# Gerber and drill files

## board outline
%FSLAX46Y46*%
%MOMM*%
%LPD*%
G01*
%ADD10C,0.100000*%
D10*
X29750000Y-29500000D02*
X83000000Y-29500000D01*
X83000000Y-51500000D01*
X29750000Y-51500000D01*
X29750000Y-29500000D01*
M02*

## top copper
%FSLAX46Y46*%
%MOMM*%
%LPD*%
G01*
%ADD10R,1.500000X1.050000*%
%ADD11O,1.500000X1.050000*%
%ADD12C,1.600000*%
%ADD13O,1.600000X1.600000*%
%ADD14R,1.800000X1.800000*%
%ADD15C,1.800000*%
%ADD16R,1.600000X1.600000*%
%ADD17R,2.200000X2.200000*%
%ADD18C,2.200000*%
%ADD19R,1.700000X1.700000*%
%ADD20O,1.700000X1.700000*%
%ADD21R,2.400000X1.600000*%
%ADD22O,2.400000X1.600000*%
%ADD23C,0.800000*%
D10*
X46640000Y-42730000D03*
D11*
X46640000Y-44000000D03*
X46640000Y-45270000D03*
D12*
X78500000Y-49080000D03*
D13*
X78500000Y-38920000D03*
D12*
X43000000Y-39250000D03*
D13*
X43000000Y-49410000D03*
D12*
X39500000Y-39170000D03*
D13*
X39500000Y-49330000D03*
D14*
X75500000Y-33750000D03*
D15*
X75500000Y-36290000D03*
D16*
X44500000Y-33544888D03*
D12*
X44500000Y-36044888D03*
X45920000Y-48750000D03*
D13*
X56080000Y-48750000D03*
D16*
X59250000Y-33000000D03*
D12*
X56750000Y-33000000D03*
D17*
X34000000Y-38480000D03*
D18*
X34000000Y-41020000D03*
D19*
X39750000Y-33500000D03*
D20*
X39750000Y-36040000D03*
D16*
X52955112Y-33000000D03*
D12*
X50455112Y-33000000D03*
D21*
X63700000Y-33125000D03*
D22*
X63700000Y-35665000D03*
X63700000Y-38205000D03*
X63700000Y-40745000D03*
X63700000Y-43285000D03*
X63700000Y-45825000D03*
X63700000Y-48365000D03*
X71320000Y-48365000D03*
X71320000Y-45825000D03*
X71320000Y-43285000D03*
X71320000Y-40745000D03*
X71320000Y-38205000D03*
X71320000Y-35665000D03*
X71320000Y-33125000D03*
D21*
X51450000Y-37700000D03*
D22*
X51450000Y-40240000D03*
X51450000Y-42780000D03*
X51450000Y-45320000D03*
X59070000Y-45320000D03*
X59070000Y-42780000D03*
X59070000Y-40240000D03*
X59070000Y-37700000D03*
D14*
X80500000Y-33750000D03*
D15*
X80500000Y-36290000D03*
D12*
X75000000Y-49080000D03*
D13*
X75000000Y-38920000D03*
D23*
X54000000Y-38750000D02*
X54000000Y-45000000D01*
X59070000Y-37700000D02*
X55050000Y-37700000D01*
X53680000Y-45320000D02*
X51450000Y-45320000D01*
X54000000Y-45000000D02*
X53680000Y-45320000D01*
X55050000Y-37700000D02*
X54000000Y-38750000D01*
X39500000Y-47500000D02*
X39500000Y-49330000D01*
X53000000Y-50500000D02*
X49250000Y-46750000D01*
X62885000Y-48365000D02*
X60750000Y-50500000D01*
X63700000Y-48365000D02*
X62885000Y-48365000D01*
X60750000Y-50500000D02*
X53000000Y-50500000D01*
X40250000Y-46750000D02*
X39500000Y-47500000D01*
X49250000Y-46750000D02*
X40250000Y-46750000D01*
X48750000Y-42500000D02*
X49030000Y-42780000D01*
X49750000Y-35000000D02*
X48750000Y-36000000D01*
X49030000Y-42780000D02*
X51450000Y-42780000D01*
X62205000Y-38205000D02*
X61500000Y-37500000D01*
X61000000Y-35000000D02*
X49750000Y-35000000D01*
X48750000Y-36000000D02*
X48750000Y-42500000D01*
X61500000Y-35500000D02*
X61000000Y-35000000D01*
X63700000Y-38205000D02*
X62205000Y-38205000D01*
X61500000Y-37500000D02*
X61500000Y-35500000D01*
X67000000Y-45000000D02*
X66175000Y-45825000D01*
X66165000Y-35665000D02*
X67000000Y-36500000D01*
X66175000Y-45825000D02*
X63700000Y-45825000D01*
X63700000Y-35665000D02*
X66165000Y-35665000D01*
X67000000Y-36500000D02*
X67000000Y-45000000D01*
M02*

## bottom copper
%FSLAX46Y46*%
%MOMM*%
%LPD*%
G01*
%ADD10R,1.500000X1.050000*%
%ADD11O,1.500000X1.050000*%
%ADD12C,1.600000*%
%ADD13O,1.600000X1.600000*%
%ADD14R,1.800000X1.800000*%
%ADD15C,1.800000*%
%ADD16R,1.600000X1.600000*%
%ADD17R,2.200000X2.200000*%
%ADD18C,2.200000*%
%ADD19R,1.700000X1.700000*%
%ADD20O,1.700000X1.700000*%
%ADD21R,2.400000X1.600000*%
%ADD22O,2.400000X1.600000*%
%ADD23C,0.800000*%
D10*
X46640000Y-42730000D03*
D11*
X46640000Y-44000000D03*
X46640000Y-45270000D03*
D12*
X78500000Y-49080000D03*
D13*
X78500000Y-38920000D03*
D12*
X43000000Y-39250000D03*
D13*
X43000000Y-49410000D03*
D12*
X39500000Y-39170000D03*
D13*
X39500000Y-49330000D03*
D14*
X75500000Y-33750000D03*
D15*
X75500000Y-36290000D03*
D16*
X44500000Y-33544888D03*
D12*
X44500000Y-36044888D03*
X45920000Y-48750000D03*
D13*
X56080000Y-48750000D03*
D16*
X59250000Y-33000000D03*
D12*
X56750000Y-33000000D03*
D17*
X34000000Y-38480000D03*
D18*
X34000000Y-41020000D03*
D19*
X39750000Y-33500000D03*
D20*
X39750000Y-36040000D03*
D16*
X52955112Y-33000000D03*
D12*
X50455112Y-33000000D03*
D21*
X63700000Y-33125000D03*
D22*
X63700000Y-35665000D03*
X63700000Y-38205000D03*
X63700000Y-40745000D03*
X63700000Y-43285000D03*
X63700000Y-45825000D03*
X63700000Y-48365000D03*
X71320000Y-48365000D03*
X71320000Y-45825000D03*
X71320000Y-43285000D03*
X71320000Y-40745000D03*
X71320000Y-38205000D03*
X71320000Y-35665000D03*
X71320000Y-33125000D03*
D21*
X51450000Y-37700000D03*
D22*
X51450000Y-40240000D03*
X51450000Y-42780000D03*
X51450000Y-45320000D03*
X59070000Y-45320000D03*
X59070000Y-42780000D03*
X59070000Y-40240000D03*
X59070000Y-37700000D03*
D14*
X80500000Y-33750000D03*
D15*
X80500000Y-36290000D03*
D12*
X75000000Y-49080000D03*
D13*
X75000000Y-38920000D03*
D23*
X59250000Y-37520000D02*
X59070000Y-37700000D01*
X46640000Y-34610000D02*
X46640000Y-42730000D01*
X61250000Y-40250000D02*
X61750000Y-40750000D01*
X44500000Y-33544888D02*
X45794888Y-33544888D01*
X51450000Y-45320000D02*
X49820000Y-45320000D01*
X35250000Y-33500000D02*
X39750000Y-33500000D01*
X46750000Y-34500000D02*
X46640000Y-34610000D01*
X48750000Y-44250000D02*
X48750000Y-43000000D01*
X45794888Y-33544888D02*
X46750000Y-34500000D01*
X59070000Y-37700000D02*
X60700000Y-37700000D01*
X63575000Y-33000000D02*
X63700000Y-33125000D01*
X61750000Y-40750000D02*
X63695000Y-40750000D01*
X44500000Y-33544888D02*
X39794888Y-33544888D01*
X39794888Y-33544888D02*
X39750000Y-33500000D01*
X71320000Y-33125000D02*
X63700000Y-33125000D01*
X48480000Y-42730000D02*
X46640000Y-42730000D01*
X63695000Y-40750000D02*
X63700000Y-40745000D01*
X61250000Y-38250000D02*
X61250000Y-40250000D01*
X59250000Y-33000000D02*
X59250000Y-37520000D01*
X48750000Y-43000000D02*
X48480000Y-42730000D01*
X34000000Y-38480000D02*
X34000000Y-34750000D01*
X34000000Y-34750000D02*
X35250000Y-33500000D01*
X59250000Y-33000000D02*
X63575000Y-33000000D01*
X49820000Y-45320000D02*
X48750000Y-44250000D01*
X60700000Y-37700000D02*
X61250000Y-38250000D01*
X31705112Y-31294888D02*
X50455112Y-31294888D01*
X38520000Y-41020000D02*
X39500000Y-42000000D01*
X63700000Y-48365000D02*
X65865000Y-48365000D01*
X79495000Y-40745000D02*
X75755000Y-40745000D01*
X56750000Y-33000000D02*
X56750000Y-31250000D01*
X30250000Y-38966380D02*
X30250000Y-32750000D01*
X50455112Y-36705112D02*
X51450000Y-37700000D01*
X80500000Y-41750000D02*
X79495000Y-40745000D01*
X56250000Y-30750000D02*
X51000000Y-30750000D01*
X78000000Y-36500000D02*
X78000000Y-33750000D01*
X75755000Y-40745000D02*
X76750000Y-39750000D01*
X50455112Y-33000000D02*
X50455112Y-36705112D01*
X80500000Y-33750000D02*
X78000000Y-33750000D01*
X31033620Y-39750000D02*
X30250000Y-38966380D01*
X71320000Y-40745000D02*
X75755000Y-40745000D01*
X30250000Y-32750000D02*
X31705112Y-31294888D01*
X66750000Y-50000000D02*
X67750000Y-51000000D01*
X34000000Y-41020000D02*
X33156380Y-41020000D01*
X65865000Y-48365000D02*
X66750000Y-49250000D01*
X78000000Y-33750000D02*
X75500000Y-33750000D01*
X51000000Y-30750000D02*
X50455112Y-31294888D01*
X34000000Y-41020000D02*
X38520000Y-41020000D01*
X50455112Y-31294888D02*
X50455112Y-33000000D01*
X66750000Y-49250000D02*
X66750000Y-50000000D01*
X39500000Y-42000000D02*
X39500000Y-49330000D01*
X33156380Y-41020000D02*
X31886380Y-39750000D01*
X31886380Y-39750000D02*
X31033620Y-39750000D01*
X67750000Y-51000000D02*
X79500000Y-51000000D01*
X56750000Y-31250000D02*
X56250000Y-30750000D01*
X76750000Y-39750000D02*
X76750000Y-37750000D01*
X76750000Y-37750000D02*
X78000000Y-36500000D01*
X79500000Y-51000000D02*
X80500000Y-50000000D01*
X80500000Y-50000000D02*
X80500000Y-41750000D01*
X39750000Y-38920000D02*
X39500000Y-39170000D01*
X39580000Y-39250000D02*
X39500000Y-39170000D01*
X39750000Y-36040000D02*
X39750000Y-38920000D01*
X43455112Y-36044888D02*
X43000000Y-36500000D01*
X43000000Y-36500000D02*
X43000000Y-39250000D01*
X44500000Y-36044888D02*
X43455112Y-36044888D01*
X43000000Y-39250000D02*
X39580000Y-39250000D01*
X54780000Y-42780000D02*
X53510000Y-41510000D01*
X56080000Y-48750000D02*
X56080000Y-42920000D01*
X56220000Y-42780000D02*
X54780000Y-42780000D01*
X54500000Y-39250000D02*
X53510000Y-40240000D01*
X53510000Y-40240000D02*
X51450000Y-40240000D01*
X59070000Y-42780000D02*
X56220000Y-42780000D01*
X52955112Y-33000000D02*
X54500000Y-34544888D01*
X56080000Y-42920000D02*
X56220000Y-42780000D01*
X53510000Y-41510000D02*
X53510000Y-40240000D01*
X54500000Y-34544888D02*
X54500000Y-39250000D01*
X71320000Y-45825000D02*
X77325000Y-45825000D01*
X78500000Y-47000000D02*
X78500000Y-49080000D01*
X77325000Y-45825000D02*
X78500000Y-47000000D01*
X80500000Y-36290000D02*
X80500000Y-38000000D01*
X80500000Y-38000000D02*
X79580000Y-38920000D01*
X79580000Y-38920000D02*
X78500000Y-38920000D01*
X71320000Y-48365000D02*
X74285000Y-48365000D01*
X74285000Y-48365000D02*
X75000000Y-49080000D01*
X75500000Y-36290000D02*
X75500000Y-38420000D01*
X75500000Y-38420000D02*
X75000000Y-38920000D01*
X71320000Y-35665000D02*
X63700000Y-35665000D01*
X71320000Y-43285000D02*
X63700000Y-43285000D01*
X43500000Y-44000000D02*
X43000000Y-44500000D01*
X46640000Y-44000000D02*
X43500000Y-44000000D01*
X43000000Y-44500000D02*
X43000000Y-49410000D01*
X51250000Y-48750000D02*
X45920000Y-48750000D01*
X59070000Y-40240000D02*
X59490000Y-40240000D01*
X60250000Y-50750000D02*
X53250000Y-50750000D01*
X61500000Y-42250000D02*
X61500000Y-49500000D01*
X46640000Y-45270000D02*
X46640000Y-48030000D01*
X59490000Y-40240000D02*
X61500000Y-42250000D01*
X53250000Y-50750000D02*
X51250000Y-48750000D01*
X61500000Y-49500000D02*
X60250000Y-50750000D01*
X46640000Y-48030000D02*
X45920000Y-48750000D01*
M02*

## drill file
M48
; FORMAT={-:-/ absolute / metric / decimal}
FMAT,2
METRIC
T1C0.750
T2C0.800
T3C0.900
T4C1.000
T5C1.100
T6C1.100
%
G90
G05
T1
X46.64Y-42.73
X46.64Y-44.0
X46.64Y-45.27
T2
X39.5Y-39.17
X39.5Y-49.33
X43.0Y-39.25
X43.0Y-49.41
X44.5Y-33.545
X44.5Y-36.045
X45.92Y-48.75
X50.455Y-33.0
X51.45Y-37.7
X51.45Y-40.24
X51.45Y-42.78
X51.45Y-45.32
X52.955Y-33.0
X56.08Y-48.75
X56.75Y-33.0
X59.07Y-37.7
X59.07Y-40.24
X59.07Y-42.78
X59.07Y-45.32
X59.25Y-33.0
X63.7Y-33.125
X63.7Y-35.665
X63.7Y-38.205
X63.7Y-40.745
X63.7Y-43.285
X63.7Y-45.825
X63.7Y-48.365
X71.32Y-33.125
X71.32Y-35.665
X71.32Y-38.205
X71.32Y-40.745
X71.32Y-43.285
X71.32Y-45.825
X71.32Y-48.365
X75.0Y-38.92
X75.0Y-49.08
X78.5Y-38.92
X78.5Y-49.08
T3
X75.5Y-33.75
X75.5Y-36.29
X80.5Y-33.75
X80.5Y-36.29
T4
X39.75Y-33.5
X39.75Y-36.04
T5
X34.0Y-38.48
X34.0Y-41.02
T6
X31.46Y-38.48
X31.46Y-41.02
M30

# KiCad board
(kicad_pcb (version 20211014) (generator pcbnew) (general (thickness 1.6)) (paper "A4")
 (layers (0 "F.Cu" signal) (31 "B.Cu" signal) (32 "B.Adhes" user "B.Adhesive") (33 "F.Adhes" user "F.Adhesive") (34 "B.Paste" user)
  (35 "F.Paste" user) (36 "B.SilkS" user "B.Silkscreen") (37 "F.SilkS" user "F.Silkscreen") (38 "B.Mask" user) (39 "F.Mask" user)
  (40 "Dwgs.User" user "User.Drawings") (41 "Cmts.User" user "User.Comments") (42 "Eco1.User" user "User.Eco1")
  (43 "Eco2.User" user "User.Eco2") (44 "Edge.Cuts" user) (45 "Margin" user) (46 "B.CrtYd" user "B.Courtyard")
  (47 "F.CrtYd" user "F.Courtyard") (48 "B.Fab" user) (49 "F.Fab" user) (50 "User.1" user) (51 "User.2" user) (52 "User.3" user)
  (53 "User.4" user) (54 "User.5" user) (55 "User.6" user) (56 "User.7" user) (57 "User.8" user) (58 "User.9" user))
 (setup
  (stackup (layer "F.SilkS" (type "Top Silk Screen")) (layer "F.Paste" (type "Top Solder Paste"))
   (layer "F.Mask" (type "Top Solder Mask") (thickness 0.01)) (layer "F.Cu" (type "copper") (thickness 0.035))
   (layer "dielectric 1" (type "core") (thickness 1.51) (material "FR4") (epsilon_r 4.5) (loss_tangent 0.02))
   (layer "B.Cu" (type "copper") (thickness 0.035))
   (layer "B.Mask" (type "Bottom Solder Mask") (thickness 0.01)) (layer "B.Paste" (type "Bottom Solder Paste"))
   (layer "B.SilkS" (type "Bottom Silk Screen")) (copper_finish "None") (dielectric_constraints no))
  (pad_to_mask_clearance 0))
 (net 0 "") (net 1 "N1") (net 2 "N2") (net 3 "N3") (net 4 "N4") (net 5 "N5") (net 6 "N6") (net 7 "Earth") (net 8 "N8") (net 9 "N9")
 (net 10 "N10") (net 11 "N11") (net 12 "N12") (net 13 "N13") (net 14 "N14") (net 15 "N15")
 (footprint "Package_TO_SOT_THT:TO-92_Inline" (layer "F.Cu") (at 46.64 42.73 -90)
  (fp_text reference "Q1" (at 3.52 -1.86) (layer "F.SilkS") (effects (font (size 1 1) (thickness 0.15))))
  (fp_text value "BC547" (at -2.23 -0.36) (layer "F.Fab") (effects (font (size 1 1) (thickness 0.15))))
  (pad "1" thru_hole rect locked (at 0 0 270) (size 1.05 1.5) (drill 0.75) (layers *.Cu *.Mask) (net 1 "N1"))
  (pad "2" thru_hole oval locked (at 1.27 0 270) (size 1.05 1.5) (drill 0.75) (layers *.Cu *.Mask) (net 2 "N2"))
  (pad "3" thru_hole oval locked (at 2.54 0 270) (size 1.05 1.5) (drill 0.75) (layers *.Cu *.Mask) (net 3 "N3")))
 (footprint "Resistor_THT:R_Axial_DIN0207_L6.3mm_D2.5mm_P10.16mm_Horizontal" (layer "F.Cu") (at 78.5 49.08 90)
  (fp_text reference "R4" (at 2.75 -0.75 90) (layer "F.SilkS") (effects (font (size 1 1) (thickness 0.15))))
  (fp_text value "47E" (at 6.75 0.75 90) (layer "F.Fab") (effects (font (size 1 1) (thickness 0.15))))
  (pad "1" thru_hole circle locked (at 0 0 90) (size 1.6 1.6) (drill 0.8) (layers *.Cu *.Mask) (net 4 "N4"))
  (pad "2" thru_hole oval locked (at 10.16 0 90) (size 1.6 1.6) (drill 0.8) (layers *.Cu *.Mask) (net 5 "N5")))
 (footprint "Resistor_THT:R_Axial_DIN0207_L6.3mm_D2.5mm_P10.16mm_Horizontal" (layer "F.Cu") (at 43 39.25 -90)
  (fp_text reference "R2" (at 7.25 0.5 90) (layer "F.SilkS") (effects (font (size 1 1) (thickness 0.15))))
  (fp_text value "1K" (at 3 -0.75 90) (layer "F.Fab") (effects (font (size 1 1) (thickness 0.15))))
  (pad "1" thru_hole circle locked (at 0 0 270) (size 1.6 1.6) (drill 0.8) (layers *.Cu *.Mask) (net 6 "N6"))
  (pad "2" thru_hole oval locked (at 10.16 0 270) (size 1.6 1.6) (drill 0.8) (layers *.Cu *.Mask) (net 2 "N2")))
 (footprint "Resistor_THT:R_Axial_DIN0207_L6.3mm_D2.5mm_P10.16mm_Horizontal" (layer "F.Cu") (at 39.5 39.17 -90)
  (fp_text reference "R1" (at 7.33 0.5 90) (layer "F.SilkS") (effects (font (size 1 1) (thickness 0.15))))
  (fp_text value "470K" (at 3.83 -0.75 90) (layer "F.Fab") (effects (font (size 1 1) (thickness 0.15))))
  (pad "1" thru_hole circle locked (at 0 0 270) (size 1.6 1.6) (drill 0.8) (layers *.Cu *.Mask) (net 6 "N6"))
  (pad "2" thru_hole oval locked (at 10.16 0 270) (size 1.6 1.6) (drill 0.8) (layers *.Cu *.Mask) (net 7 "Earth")))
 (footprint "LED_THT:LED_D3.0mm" (layer "F.Cu") (at 75.5 33.75 -90)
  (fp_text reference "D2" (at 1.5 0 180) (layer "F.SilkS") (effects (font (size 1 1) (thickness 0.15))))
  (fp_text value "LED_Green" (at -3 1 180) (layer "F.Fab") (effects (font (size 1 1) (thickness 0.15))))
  (pad "1" thru_hole rect locked (at 0 0 270) (size 1.8 1.8) (drill 0.9) (layers *.Cu *.Mask) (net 7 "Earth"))
  (pad "2" thru_hole circle locked (at 2.54 0 270) (size 1.8 1.8) (drill 0.9) (layers *.Cu *.Mask) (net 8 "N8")))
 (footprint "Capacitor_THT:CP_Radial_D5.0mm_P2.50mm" (layer "F.Cu") (at 44.5 33.544888 -90)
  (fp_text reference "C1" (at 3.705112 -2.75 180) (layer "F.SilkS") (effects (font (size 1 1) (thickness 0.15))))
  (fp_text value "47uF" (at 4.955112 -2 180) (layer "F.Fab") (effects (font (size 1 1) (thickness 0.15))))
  (pad "1" thru_hole rect locked (at 0 0 270) (size 1.6 1.6) (drill 0.8) (layers *.Cu *.Mask) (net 1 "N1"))
  (pad "2" thru_hole circle locked (at 2.5 0 270) (size 1.6 1.6) (drill 0.8) (layers *.Cu *.Mask) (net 6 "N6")))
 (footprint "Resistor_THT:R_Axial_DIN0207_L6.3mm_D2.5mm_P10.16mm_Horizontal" (layer "F.Cu") (at 45.92 48.75)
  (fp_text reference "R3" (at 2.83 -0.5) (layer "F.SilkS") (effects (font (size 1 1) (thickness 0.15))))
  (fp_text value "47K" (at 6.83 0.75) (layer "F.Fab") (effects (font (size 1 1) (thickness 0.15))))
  (pad "1" thru_hole circle locked (at 0 0) (size 1.6 1.6) (drill 0.8) (layers *.Cu *.Mask) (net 3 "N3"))
  (pad "2" thru_hole oval locked (at 10.16 0) (size 1.6 1.6) (drill 0.8) (layers *.Cu *.Mask) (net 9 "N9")))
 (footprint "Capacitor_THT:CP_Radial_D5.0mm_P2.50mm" (layer "F.Cu") (at 59.25 33 180)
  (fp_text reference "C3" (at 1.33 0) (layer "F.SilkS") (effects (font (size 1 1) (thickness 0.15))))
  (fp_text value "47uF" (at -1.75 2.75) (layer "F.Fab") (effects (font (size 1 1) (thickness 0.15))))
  (pad "1" thru_hole rect locked (at 0 0 180) (size 1.6 1.6) (drill 0.8) (layers *.Cu *.Mask) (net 1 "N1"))
  (pad "2" thru_hole circle locked (at 2.5 0 180) (size 1.6 1.6) (drill 0.8) (layers *.Cu *.Mask) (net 7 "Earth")))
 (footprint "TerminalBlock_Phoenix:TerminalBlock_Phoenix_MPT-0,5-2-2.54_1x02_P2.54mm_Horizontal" (layer "F.Cu") (at 34 38.48 -90)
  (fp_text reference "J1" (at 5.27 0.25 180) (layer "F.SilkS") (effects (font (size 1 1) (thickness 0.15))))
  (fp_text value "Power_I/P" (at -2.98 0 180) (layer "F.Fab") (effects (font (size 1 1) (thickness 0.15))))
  (pad "" np_thru_hole circle locked (at 2.54 2.54 270) (size 1.1 1.1) (drill 1.1) (layers *.Cu *.Mask))
  (pad "" np_thru_hole circle locked (at 0 2.54 270) (size 1.1 1.1) (drill 1.1) (layers *.Cu *.Mask))
  (pad "1" thru_hole rect locked (at 0 0 270) (size 2.2 2.2) (drill 1.1) (layers *.Cu *.Mask) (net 1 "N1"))
  (pad "2" thru_hole circle locked (at 2.54 0 270) (size 2.2 2.2) (drill 1.1) (layers *.Cu *.Mask) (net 7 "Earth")))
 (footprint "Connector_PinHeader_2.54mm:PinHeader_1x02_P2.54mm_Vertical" (layer "F.Cu") (at 39.75 33.5)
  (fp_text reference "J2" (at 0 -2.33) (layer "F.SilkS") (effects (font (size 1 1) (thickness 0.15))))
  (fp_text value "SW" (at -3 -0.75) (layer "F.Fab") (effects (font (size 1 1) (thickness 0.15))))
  (pad "1" thru_hole rect locked (at 0 0) (size 1.7 1.7) (drill 1) (layers *.Cu *.Mask) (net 1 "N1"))
  (pad "2" thru_hole oval locked (at 0 2.54) (size 1.7 1.7) (drill 1) (layers *.Cu *.Mask) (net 6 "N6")))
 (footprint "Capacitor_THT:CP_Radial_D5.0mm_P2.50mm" (layer "F.Cu") (at 52.955112 33 180)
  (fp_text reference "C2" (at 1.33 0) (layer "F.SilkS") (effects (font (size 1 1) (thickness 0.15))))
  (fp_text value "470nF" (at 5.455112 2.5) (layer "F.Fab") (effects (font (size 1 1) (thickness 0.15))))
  (pad "1" thru_hole rect locked (at 0 0 180) (size 1.6 1.6) (drill 0.8) (layers *.Cu *.Mask) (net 9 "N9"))
  (pad "2" thru_hole circle locked (at 2.5 0 180) (size 1.6 1.6) (drill 0.8) (layers *.Cu *.Mask) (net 7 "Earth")))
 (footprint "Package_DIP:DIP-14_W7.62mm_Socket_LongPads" (layer "F.Cu") (at 63.7 33.125)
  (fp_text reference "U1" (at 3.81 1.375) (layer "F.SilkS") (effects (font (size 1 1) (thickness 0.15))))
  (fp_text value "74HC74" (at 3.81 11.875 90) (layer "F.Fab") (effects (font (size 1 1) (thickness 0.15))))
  (pad "1" thru_hole rect locked (at 0 0) (size 2.4 1.6) (drill 0.8) (layers *.Cu *.Mask) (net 1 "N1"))
  (pad "2" thru_hole oval locked (at 0 2.54) (size 2.4 1.6) (drill 0.8) (layers *.Cu *.Mask) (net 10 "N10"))
  (pad "3" thru_hole oval locked (at 0 5.08) (size 2.4 1.6) (drill 0.8) (layers *.Cu *.Mask) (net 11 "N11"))
  (pad "4" thru_hole oval locked (at 0 7.62) (size 2.4 1.6) (drill 0.8) (layers *.Cu *.Mask) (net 1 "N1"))
  (pad "5" thru_hole oval locked (at 0 10.16) (size 2.4 1.6) (drill 0.8) (layers *.Cu *.Mask) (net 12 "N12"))
  (pad "6" thru_hole oval locked (at 0 12.7) (size 2.4 1.6) (drill 0.8) (layers *.Cu *.Mask) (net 10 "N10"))
  (pad "7" thru_hole oval locked (at 0 15.24) (size 2.4 1.6) (drill 0.8) (layers *.Cu *.Mask) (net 7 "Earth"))
  (pad "8" thru_hole oval locked (at 7.62 15.24) (size 2.4 1.6) (drill 0.8) (layers *.Cu *.Mask) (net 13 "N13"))
  (pad "9" thru_hole oval locked (at 7.62 12.7) (size 2.4 1.6) (drill 0.8) (layers *.Cu *.Mask) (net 4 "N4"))
  (pad "10" thru_hole oval locked (at 7.62 10.16) (size 2.4 1.6) (drill 0.8) (layers *.Cu *.Mask) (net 12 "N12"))
  (pad "11" thru_hole oval locked (at 7.62 7.62) (size 2.4 1.6) (drill 0.8) (layers *.Cu *.Mask) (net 7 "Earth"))
  (pad "12" thru_hole oval locked (at 7.62 5.08) (size 2.4 1.6) (drill 0.8) (layers *.Cu *.Mask) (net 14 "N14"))
  (pad "13" thru_hole oval locked (at 7.62 2.54) (size 2.4 1.6) (drill 0.8) (layers *.Cu *.Mask) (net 10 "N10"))
  (pad "14" thru_hole oval locked (at 7.62 0) (size 2.4 1.6) (drill 0.8) (layers *.Cu *.Mask) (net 1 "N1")))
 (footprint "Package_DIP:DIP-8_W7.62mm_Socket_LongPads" (layer "F.Cu") (at 51.45 37.7)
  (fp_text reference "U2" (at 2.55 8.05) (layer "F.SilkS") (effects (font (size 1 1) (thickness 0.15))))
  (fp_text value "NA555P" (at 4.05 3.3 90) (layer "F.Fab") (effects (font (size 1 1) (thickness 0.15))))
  (pad "1" thru_hole rect locked (at 0 0) (size 2.4 1.6) (drill 0.8) (layers *.Cu *.Mask) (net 7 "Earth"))
  (pad "2" thru_hole oval locked (at 0 2.54) (size 2.4 1.6) (drill 0.8) (layers *.Cu *.Mask) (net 9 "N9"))
  (pad "3" thru_hole oval locked (at 0 5.08) (size 2.4 1.6) (drill 0.8) (layers *.Cu *.Mask) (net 11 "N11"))
  (pad "4" thru_hole oval locked (at 0 7.62) (size 2.4 1.6) (drill 0.8) (layers *.Cu *.Mask) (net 1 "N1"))
  (pad "5" thru_hole oval locked (at 7.62 7.62) (size 2.4 1.6) (drill 0.8) (layers *.Cu *.Mask) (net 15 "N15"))
  (pad "6" thru_hole oval locked (at 7.62 5.08) (size 2.4 1.6) (drill 0.8) (layers *.Cu *.Mask) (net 9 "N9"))
  (pad "7" thru_hole oval locked (at 7.62 2.54) (size 2.4 1.6) (drill 0.8) (layers *.Cu *.Mask) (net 3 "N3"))
  (pad "8" thru_hole oval locked (at 7.62 0) (size 2.4 1.6) (drill 0.8) (layers *.Cu *.Mask) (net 1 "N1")))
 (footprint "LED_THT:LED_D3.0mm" (layer "F.Cu") (at 80.5 33.75 -90)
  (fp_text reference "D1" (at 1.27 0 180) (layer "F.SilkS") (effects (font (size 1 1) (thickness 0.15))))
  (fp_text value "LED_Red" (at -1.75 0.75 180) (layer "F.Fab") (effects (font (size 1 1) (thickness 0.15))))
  (pad "1" thru_hole rect locked (at 0 0 270) (size 1.8 1.8) (drill 0.9) (layers *.Cu *.Mask) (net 7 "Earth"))
  (pad "2" thru_hole circle locked (at 2.54 0 270) (size 1.8 1.8) (drill 0.9) (layers *.Cu *.Mask) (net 5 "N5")))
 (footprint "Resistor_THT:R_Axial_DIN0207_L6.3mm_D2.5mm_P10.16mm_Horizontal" (layer "F.Cu") (at 75 49.08 90)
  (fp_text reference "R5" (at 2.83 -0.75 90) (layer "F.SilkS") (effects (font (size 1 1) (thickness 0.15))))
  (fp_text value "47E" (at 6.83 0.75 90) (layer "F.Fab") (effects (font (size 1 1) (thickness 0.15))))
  (pad "1" thru_hole circle locked (at 0 0 90) (size 1.6 1.6) (drill 0.8) (layers *.Cu *.Mask) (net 13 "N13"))
  (pad "2" thru_hole oval locked (at 10.16 0 90) (size 1.6 1.6) (drill 0.8) (layers *.Cu *.Mask) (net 8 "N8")))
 (gr_rect (start 29.75 29.5) (end 83 51.5) (layer "Edge.Cuts") (width 0.1) (fill none))
 (segment (start 54 38.75) (end 54 45) (width 0.8) (layer "F.Cu") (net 1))
 (segment (start 59.07 37.7) (end 55.05 37.7) (width 0.8) (layer "F.Cu") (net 1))
 (segment (start 53.68 45.32) (end 51.45 45.32) (width 0.8) (layer "F.Cu") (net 1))
 (segment (start 54 45) (end 53.68 45.32) (width 0.8) (layer "F.Cu") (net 1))
 (segment (start 55.05 37.7) (end 54 38.75) (width 0.8) (layer "F.Cu") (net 1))
 (segment (start 59.25 37.52) (end 59.07 37.7) (width 0.8) (layer "B.Cu") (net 1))
 (segment (start 46.64 34.61) (end 46.64 42.73) (width 0.8) (layer "B.Cu") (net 1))
 (segment (start 61.25 40.25) (end 61.75 40.75) (width 0.8) (layer "B.Cu") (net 1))
 (segment (start 44.5 33.544888) (end 45.794888 33.544888) (width 0.8) (layer "B.Cu") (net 1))
 (segment (start 51.45 45.32) (end 49.82 45.32) (width 0.8) (layer "B.Cu") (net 1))
 (segment (start 35.25 33.5) (end 39.75 33.5) (width 0.8) (layer "B.Cu") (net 1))
 (segment (start 46.75 34.5) (end 46.64 34.61) (width 0.8) (layer "B.Cu") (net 1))
 (segment (start 48.75 44.25) (end 48.75 43) (width 0.8) (layer "B.Cu") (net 1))
 (segment (start 45.794888 33.544888) (end 46.75 34.5) (width 0.8) (layer "B.Cu") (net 1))
 (segment (start 59.07 37.7) (end 60.7 37.7) (width 0.8) (layer "B.Cu") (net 1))
 (segment (start 63.575 33) (end 63.7 33.125) (width 0.8) (layer "B.Cu") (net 1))
 (segment (start 61.75 40.75) (end 63.695 40.75) (width 0.8) (layer "B.Cu") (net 1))
 (segment (start 44.5 33.544888) (end 39.794888 33.544888) (width 0.8) (layer "B.Cu") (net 1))
 (segment (start 39.794888 33.544888) (end 39.75 33.5) (width 0.8) (layer "B.Cu") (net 1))
 (segment (start 71.32 33.125) (end 63.7 33.125) (width 0.8) (layer "B.Cu") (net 1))
 (segment (start 48.48 42.73) (end 46.64 42.73) (width 0.8) (layer "B.Cu") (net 1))
 (segment (start 63.695 40.75) (end 63.7 40.745) (width 0.8) (layer "B.Cu") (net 1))
 (segment (start 61.25 38.25) (end 61.25 40.25) (width 0.8) (layer "B.Cu") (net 1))
 (segment (start 59.25 33) (end 59.25 37.52) (width 0.8) (layer "B.Cu") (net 1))
 (segment (start 48.75 43) (end 48.48 42.73) (width 0.8) (layer "B.Cu") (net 1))
 (segment (start 34 38.48) (end 34 34.75) (width 0.8) (layer "B.Cu") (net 1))
 (segment (start 34 34.75) (end 35.25 33.5) (width 0.8) (layer "B.Cu") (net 1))
 (segment (start 59.25 33) (end 63.575 33) (width 0.8) (layer "B.Cu") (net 1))
 (segment (start 49.82 45.32) (end 48.75 44.25) (width 0.8) (layer "B.Cu") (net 1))
 (segment (start 60.7 37.7) (end 61.25 38.25) (width 0.8) (layer "B.Cu") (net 1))
 (segment (start 39.5 47.5) (end 39.5 49.33) (width 0.8) (layer "F.Cu") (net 7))
 (segment (start 53 50.5) (end 49.25 46.75) (width 0.8) (layer "F.Cu") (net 7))
 (segment (start 62.885 48.365) (end 60.75 50.5) (width 0.8) (layer "F.Cu") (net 7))
 (segment (start 63.7 48.365) (end 62.885 48.365) (width 0.8) (layer "F.Cu") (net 7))
 (segment (start 60.75 50.5) (end 53 50.5) (width 0.8) (layer "F.Cu") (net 7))
 (segment (start 40.25 46.75) (end 39.5 47.5) (width 0.8) (layer "F.Cu") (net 7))
 (segment (start 49.25 46.75) (end 40.25 46.75) (width 0.8) (layer "F.Cu") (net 7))
 (segment (start 31.705112 31.294888) (end 50.455112 31.294888) (width 0.8) (layer "B.Cu") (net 7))
 (segment (start 38.52 41.02) (end 39.5 42) (width 0.8) (layer "B.Cu") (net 7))
 (segment (start 63.7 48.365) (end 65.865 48.365) (width 0.8) (layer "B.Cu") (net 7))
 (segment (start 79.495 40.745) (end 75.755 40.745) (width 0.8) (layer "B.Cu") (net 7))
 (segment (start 56.75 33) (end 56.75 31.25) (width 0.8) (layer "B.Cu") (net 7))
 (segment (start 30.25 38.96638) (end 30.25 32.75) (width 0.8) (layer "B.Cu") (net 7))
 (segment (start 50.455112 36.705112) (end 51.45 37.7) (width 0.8) (layer "B.Cu") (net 7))
 (segment (start 80.5 41.75) (end 79.495 40.745) (width 0.8) (layer "B.Cu") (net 7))
 (segment (start 56.25 30.75) (end 51 30.75) (width 0.8) (layer "B.Cu") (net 7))
 (segment (start 78 36.5) (end 78 33.75) (width 0.8) (layer "B.Cu") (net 7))
 (segment (start 75.755 40.745) (end 76.75 39.75) (width 0.8) (layer "B.Cu") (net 7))
 (segment (start 50.455112 33) (end 50.455112 36.705112) (width 0.8) (layer "B.Cu") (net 7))
 (segment (start 80.5 33.75) (end 78 33.75) (width 0.8) (layer "B.Cu") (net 7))
 (segment (start 31.03362 39.75) (end 30.25 38.96638) (width 0.8) (layer "B.Cu") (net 7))
 (segment (start 71.32 40.745) (end 75.755 40.745) (width 0.8) (layer "B.Cu") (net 7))
 (segment (start 30.25 32.75) (end 31.705112 31.294888) (width 0.8) (layer "B.Cu") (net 7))
 (segment (start 66.75 50) (end 67.75 51) (width 0.8) (layer "B.Cu") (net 7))
 (segment (start 34 41.02) (end 33.15638 41.02) (width 0.8) (layer "B.Cu") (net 7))
 (segment (start 65.865 48.365) (end 66.75 49.25) (width 0.8) (layer "B.Cu") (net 7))
 (segment (start 78 33.75) (end 75.5 33.75) (width 0.8) (layer "B.Cu") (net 7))
 (segment (start 51 30.75) (end 50.455112 31.294888) (width 0.8) (layer "B.Cu") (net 7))
 (segment (start 34 41.02) (end 38.52 41.02) (width 0.8) (layer "B.Cu") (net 7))
 (segment (start 50.455112 31.294888) (end 50.455112 33) (width 0.8) (layer "B.Cu") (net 7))
 (segment (start 66.75 49.25) (end 66.75 50) (width 0.8) (layer "B.Cu") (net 7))
 (segment (start 39.5 42) (end 39.5 49.33) (width 0.8) (layer "B.Cu") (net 7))
 (segment (start 33.15638 41.02) (end 31.88638 39.75) (width 0.8) (layer "B.Cu") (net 7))
 (segment (start 31.88638 39.75) (end 31.03362 39.75) (width 0.8) (layer "B.Cu") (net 7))
 (segment (start 67.75 51) (end 79.5 51) (width 0.8) (layer "B.Cu") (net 7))
 (segment (start 56.75 31.25) (end 56.25 30.75) (width 0.8) (layer "B.Cu") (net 7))
 (segment (start 76.75 39.75) (end 76.75 37.75) (width 0.8) (layer "B.Cu") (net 7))
 (segment (start 76.75 37.75) (end 78 36.5) (width 0.8) (layer "B.Cu") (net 7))
 (segment (start 79.5 51) (end 80.5 50) (width 0.8) (layer "B.Cu") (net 7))
 (segment (start 80.5 50) (end 80.5 41.75) (width 0.8) (layer "B.Cu") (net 7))
 (segment (start 39.75 38.92) (end 39.5 39.17) (width 0.8) (layer "B.Cu") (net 6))
 (segment (start 39.58 39.25) (end 39.5 39.17) (width 0.8) (layer "B.Cu") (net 6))
 (segment (start 39.75 36.04) (end 39.75 38.92) (width 0.8) (layer "B.Cu") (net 6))
 (segment (start 43.455112 36.044888) (end 43 36.5) (width 0.8) (layer "B.Cu") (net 6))
 (segment (start 43 36.5) (end 43 39.25) (width 0.8) (layer "B.Cu") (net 6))
 (segment (start 44.5 36.044888) (end 43.455112 36.044888) (width 0.8) (layer "B.Cu") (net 6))
 (segment (start 43 39.25) (end 39.58 39.25) (width 0.8) (layer "B.Cu") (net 6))
 (segment (start 54.78 42.78) (end 53.51 41.51) (width 0.8) (layer "B.Cu") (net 9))
 (segment (start 56.08 48.75) (end 56.08 42.92) (width 0.8) (layer "B.Cu") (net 9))
 (segment (start 56.22 42.78) (end 54.78 42.78) (width 0.8) (layer "B.Cu") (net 9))
 (segment (start 54.5 39.25) (end 53.51 40.24) (width 0.8) (layer "B.Cu") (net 9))
 (segment (start 53.51 40.24) (end 51.45 40.24) (width 0.8) (layer "B.Cu") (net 9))
 (segment (start 59.07 42.78) (end 56.22 42.78) (width 0.8) (layer "B.Cu") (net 9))
 (segment (start 52.955112 33) (end 54.5 34.544888) (width 0.8) (layer "B.Cu") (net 9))
 (segment (start 56.08 42.92) (end 56.22 42.78) (width 0.8) (layer "B.Cu") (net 9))
 (segment (start 53.51 41.51) (end 53.51 40.24) (width 0.8) (layer "B.Cu") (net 9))
 (segment (start 54.5 34.544888) (end 54.5 39.25) (width 0.8) (layer "B.Cu") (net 9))
 (segment (start 71.32 45.825) (end 77.325 45.825) (width 0.8) (layer "B.Cu") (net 4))
 (segment (start 78.5 47) (end 78.5 49.08) (width 0.8) (layer "B.Cu") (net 4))
 (segment (start 77.325 45.825) (end 78.5 47) (width 0.8) (layer "B.Cu") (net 4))
 (segment (start 80.5 36.29) (end 80.5 38) (width 0.8) (layer "B.Cu") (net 5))
 (segment (start 80.5 38) (end 79.58 38.92) (width 0.8) (layer "B.Cu") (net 5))
 (segment (start 79.58 38.92) (end 78.5 38.92) (width 0.8) (layer "B.Cu") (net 5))
 (segment (start 71.32 48.365) (end 74.285 48.365) (width 0.8) (layer "B.Cu") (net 13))
 (segment (start 74.285 48.365) (end 75 49.08) (width 0.8) (layer "B.Cu") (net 13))
 (segment (start 75.5 36.29) (end 75.5 38.42) (width 0.8) (layer "B.Cu") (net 8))
 (segment (start 75.5 38.42) (end 75 38.92) (width 0.8) (layer "B.Cu") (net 8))
 (segment (start 48.75 42.5) (end 49.03 42.78) (width 0.8) (layer "F.Cu") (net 11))
 (segment (start 49.75 35) (end 48.75 36) (width 0.8) (layer "F.Cu") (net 11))
 (segment (start 49.03 42.78) (end 51.45 42.78) (width 0.8) (layer "F.Cu") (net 11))
 (segment (start 62.205 38.205) (end 61.5 37.5) (width 0.8) (layer "F.Cu") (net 11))
 (segment (start 61 35) (end 49.75 35) (width 0.8) (layer "F.Cu") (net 11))
 (segment (start 48.75 36) (end 48.75 42.5) (width 0.8) (layer "F.Cu") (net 11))
 (segment (start 61.5 35.5) (end 61 35) (width 0.8) (layer "F.Cu") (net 11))
 (segment (start 63.7 38.205) (end 62.205 38.205) (width 0.8) (layer "F.Cu") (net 11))
 (segment (start 61.5 37.5) (end 61.5 35.5) (width 0.8) (layer "F.Cu") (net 11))
 (segment (start 67 45) (end 66.175 45.825) (width 0.8) (layer "F.Cu") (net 10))
 (segment (start 66.165 35.665) (end 67 36.5) (width 0.8) (layer "F.Cu") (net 10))
 (segment (start 66.175 45.825) (end 63.7 45.825) (width 0.8) (layer "F.Cu") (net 10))
 (segment (start 63.7 35.665) (end 66.165 35.665) (width 0.8) (layer "F.Cu") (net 10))
 (segment (start 67 36.5) (end 67 45) (width 0.8) (layer "F.Cu") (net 10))
 (segment (start 71.32 35.665) (end 63.7 35.665) (width 0.8) (layer "B.Cu") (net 10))
 (segment (start 71.32 43.285) (end 63.7 43.285) (width 0.8) (layer "B.Cu") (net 12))
 (segment (start 43.5 44) (end 43 44.5) (width 0.8) (layer "B.Cu") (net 2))
 (segment (start 46.64 44) (end 43.5 44) (width 0.8) (layer "B.Cu") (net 2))
 (segment (start 43 44.5) (end 43 49.41) (width 0.8) (layer "B.Cu") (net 2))
 (segment (start 51.25 48.75) (end 45.92 48.75) (width 0.8) (layer "B.Cu") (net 3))
 (segment (start 59.07 40.24) (end 59.49 40.24) (width 0.8) (layer "B.Cu") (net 3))
 (segment (start 60.25 50.75) (end 53.25 50.75) (width 0.8) (layer "B.Cu") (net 3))
 (segment (start 61.5 42.25) (end 61.5 49.5) (width 0.8) (layer "B.Cu") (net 3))
 (segment (start 46.64 45.27) (end 46.64 48.03) (width 0.8) (layer "B.Cu") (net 3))
 (segment (start 59.49 40.24) (end 61.5 42.25) (width 0.8) (layer "B.Cu") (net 3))
 (segment (start 53.25 50.75) (end 51.25 48.75) (width 0.8) (layer "B.Cu") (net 3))
 (segment (start 61.5 49.5) (end 60.25 50.75) (width 0.8) (layer "B.Cu") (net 3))
 (segment (start 46.64 48.03) (end 45.92 48.75) (width 0.8) (layer "B.Cu") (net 3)))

